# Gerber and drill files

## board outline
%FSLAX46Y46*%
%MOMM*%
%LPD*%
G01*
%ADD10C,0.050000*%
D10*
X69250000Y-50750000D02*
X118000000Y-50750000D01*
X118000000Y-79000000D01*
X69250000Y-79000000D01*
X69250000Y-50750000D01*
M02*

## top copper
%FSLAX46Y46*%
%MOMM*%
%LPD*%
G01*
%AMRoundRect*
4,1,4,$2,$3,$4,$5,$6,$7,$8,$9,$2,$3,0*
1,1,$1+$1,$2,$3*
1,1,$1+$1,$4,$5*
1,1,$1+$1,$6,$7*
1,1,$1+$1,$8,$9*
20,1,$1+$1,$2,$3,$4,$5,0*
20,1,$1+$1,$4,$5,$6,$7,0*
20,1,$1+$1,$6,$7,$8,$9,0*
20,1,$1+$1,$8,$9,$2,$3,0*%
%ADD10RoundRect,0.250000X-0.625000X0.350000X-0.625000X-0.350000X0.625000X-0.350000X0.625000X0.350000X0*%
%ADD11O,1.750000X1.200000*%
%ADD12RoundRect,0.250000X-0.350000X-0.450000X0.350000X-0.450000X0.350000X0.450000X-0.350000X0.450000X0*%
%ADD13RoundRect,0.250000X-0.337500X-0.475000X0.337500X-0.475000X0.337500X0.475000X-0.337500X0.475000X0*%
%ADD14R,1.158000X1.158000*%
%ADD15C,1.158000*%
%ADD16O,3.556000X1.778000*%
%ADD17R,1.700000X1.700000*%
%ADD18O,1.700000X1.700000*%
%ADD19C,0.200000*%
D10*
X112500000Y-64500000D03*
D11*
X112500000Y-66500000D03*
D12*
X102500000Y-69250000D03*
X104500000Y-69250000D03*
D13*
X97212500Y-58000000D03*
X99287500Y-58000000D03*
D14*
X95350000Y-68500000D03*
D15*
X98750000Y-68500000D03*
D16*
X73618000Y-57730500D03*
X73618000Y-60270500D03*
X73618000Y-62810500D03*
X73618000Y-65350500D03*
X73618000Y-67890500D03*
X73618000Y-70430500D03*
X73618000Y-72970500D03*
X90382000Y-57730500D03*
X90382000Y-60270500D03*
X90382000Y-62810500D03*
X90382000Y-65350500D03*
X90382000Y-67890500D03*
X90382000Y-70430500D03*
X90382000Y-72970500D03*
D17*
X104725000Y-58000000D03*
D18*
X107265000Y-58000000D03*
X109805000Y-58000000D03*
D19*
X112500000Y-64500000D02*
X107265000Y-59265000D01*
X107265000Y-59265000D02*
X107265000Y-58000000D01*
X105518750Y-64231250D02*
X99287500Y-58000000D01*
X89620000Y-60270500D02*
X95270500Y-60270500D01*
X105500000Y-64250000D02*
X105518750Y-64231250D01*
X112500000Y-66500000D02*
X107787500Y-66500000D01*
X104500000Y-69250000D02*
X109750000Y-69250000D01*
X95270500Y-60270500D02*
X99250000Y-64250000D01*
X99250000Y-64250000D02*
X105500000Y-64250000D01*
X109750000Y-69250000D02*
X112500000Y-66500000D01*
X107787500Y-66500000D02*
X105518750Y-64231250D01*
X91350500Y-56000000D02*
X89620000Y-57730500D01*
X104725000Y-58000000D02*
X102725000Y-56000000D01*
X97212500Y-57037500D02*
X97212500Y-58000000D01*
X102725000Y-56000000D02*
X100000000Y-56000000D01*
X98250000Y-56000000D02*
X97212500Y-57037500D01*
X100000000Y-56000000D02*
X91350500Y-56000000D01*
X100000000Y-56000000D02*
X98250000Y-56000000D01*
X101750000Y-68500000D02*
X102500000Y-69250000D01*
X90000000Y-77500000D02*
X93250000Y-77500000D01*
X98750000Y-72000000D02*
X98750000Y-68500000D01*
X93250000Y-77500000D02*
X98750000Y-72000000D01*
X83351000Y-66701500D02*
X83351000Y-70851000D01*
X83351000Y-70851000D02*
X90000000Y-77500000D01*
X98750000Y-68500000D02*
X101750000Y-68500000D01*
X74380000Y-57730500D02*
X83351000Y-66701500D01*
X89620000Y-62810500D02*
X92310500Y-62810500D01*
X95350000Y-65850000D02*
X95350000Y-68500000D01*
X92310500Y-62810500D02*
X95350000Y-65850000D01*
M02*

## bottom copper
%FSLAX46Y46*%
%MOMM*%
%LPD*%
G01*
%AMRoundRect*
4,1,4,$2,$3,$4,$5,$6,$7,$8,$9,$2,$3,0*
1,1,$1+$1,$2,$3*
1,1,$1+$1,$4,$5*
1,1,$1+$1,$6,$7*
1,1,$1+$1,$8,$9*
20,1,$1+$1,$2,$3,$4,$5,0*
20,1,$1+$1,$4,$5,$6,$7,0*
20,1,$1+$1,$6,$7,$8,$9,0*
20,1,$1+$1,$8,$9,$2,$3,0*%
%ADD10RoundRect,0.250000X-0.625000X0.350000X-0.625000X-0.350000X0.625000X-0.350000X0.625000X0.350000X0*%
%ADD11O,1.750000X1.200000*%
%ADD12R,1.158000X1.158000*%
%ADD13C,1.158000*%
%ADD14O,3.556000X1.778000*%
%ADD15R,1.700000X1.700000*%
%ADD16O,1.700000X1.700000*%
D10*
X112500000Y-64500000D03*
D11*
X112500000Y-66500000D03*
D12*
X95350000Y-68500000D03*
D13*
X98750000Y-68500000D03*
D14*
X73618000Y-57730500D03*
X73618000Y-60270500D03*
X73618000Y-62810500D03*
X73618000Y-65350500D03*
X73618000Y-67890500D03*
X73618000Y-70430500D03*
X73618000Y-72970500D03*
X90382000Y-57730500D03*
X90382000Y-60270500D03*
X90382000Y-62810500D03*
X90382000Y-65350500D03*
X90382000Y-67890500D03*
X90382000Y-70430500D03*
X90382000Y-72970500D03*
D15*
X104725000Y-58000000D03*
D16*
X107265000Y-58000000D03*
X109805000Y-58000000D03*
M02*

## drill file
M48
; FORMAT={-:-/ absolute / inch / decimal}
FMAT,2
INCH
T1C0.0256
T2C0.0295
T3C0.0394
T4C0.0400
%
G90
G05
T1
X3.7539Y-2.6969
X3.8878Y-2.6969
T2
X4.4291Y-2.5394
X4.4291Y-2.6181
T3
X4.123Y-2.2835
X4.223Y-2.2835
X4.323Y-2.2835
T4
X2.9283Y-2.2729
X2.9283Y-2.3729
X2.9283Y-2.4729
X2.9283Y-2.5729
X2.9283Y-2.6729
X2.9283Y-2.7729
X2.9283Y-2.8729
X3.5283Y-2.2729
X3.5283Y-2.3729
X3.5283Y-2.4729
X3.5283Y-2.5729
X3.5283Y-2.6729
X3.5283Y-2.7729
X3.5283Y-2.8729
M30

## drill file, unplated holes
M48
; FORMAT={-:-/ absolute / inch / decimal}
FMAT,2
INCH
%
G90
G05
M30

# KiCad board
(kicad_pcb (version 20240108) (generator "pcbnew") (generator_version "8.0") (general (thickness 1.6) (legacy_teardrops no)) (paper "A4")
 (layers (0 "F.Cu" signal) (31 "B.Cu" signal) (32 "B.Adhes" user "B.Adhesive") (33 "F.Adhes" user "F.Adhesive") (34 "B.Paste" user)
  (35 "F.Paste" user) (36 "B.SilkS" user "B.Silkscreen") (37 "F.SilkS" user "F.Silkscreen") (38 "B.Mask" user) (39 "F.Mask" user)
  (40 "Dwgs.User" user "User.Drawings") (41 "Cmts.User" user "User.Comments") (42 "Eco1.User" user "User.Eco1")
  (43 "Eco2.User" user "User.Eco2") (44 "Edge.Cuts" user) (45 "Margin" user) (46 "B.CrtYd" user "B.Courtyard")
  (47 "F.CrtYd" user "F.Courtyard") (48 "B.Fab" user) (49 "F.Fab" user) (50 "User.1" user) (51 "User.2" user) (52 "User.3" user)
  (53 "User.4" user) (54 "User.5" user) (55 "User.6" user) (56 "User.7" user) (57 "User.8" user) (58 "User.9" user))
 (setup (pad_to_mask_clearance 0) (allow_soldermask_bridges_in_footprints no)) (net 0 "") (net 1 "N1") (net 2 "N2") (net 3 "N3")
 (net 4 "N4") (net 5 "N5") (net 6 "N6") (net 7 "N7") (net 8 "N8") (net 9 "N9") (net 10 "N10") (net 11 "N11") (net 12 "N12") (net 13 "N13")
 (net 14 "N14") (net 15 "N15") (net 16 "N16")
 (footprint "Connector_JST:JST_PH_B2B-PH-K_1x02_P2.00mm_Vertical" (layer "F.Cu") (at 112.5 64.5 -90)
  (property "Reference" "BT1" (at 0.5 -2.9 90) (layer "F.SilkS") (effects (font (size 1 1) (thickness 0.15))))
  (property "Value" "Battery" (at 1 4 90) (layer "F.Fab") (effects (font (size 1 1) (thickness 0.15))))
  (pad "1" thru_hole roundrect (at 0 0 270) (size 1.2 1.75) (drill 0.75) (layers "*.Cu" "*.Mask") (remove_unused_layers no)
   (roundrect_rratio 0.208333) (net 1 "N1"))
  (pad "2" thru_hole oval (at 2 0 270) (size 1.2 1.75) (drill 0.75) (layers "*.Cu" "*.Mask") (remove_unused_layers no) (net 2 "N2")))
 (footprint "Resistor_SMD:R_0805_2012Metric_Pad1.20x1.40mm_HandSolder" (layer "F.Cu") (at 104 69.25)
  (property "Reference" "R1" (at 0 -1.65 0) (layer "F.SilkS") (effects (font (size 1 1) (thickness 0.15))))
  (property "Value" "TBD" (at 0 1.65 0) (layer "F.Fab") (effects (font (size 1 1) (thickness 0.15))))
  (pad "1" smd roundrect (at -1.5 0) (size 1.2 1.4) (layers "F.Cu" "F.Paste" "F.Mask") (roundrect_rratio 0.208333) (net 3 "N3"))
  (pad "2" smd roundrect (at 0.5 0) (size 1.2 1.4) (layers "F.Cu" "F.Paste" "F.Mask") (roundrect_rratio 0.208333) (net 2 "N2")))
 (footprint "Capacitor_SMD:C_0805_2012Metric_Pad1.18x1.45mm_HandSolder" (layer "F.Cu") (at 98.25 58)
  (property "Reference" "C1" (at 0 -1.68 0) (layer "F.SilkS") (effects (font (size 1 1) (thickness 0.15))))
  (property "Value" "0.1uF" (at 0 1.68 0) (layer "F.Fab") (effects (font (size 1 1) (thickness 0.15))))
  (pad "1" smd roundrect (at -1.0375 0) (size 1.175 1.45) (layers "F.Cu" "F.Paste" "F.Mask") (roundrect_rratio 0.212766) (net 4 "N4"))
  (pad "2" smd roundrect (at 1.0375 0) (size 1.175 1.45) (layers "F.Cu" "F.Paste" "F.Mask") (roundrect_rratio 0.212766) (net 2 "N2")))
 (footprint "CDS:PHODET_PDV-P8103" (layer "F.Cu") (at 97.05 68.5)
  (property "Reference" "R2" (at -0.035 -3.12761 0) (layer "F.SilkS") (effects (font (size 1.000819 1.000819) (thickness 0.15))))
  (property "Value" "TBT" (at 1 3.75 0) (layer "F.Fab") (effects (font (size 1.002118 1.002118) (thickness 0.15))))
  (pad "1" thru_hole rect (at -1.7 0) (size 1.158 1.158) (drill 0.65) (layers "*.Cu" "*.Mask") (remove_unused_layers no) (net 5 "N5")
   (solder_mask_margin 0.102))
  (pad "2" thru_hole circle (at 1.7 0) (size 1.158 1.158) (drill 0.65) (layers "*.Cu" "*.Mask") (remove_unused_layers no) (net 3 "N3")
   (solder_mask_margin 0.102)))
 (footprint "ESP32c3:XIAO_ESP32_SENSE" (layer "F.Cu") (at 82 65.3505)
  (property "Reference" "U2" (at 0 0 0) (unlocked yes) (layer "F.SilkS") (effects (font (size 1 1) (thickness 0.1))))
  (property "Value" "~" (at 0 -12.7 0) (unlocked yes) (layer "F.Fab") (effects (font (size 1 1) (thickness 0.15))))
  (pad "1" thru_hole oval (at -7.62 -7.62) (size 3.556 1.778) (drill 1.016 (offset -0.762 0)) (layers "*.Cu" "*.Mask")
   (remove_unused_layers no) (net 3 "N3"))
  (pad "2" thru_hole oval (at -7.62 -5.08) (size 3.556 1.778) (drill 1.016 (offset -0.762 0)) (layers "*.Cu" "*.Mask")
   (remove_unused_layers no) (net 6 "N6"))
  (pad "3" thru_hole oval (at -7.62 -2.54) (size 3.556 1.778) (drill 1.016 (offset -0.762 0)) (layers "*.Cu" "*.Mask")
   (remove_unused_layers no) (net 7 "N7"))
  (pad "4" thru_hole oval (at -7.62 0) (size 3.556 1.778) (drill 1.016 (offset -0.762 0)) (layers "*.Cu" "*.Mask") (remove_unused_layers no)
   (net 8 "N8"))
  (pad "5" thru_hole oval (at -7.62 2.54) (size 3.556 1.778) (drill 1.016 (offset -0.762 0)) (layers "*.Cu" "*.Mask")
   (remove_unused_layers no) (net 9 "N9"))
  (pad "6" thru_hole oval (at -7.62 5.08) (size 3.556 1.778) (drill 1.016 (offset -0.762 0)) (layers "*.Cu" "*.Mask")
   (remove_unused_layers no) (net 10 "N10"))
  (pad "7" thru_hole oval (at -7.62 7.62) (size 3.556 1.778) (drill 1.016 (offset -0.762 0)) (layers "*.Cu" "*.Mask")
   (remove_unused_layers no) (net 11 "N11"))
  (pad "8" thru_hole oval (at 7.62 -7.62) (size 3.556 1.778) (drill 1.016 (offset 0.762 0)) (layers "*.Cu" "*.Mask")
   (remove_unused_layers no) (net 4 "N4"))
  (pad "9" thru_hole oval (at 7.62 -5.08) (size 3.556 1.778) (drill 1.016 (offset 0.762 0)) (layers "*.Cu" "*.Mask")
   (remove_unused_layers no) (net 2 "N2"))
  (pad "10" thru_hole oval (at 7.62 -2.54) (size 3.556 1.778) (drill 1.016 (offset 0.762 0)) (layers "*.Cu" "*.Mask")
   (remove_unused_layers no) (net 5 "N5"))
  (pad "11" thru_hole oval (at 7.62 0) (size 3.556 1.778) (drill 1.016 (offset 0.762 0)) (layers "*.Cu" "*.Mask") (remove_unused_layers no)
   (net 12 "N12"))
  (pad "12" thru_hole oval (at 7.62 2.54) (size 3.556 1.778) (drill 1.016 (offset 0.762 0)) (layers "*.Cu" "*.Mask")
   (remove_unused_layers no) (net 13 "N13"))
  (pad "13" thru_hole oval (at 7.62 5.08) (size 3.556 1.778) (drill 1.016 (offset 0.762 0)) (layers "*.Cu" "*.Mask")
   (remove_unused_layers no) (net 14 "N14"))
  (pad "14" thru_hole oval (at 7.62 7.62) (size 3.556 1.778) (drill 1.016 (offset 0.762 0)) (layers "*.Cu" "*.Mask")
   (remove_unused_layers no) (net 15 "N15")))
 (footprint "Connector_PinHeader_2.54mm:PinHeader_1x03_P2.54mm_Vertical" (layer "F.Cu") (at 104.725 58 90)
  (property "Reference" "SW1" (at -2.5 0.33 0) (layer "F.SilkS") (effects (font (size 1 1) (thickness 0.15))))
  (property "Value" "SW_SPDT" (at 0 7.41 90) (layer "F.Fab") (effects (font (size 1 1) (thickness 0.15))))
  (pad "1" thru_hole rect (at 0 0 90) (size 1.7 1.7) (drill 1) (layers "*.Cu" "*.Mask") (remove_unused_layers no) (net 4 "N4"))
  (pad "2" thru_hole oval (at 0 2.54 90) (size 1.7 1.7) (drill 1) (layers "*.Cu" "*.Mask") (remove_unused_layers no) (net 1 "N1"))
  (pad "3" thru_hole oval (at 0 5.08 90) (size 1.7 1.7) (drill 1) (layers "*.Cu" "*.Mask") (remove_unused_layers no) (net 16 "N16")))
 (gr_rect (start 69.25 50.75) (end 118 79) (stroke (width 0.05) (type default)) (fill none) (layer "Edge.Cuts"))
 (segment (start 112.5 64.5) (end 107.265 59.265) (width 0.2) (layer "F.Cu") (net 1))
 (segment (start 107.265 59.265) (end 107.265 58) (width 0.2) (layer "F.Cu") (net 1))
 (segment (start 105.51875 64.23125) (end 99.2875 58) (width 0.2) (layer "F.Cu") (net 2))
 (segment (start 89.62 60.2705) (end 95.2705 60.2705) (width 0.2) (layer "F.Cu") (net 2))
 (segment (start 105.5 64.25) (end 105.51875 64.23125) (width 0.2) (layer "F.Cu") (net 2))
 (segment (start 112.5 66.5) (end 107.7875 66.5) (width 0.2) (layer "F.Cu") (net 2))
 (segment (start 104.5 69.25) (end 109.75 69.25) (width 0.2) (layer "F.Cu") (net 2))
 (segment (start 95.2705 60.2705) (end 99.25 64.25) (width 0.2) (layer "F.Cu") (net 2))
 (segment (start 99.25 64.25) (end 105.5 64.25) (width 0.2) (layer "F.Cu") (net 2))
 (segment (start 109.75 69.25) (end 112.5 66.5) (width 0.2) (layer "F.Cu") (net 2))
 (segment (start 107.7875 66.5) (end 105.51875 64.23125) (width 0.2) (layer "F.Cu") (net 2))
 (segment (start 91.3505 56) (end 89.62 57.7305) (width 0.2) (layer "F.Cu") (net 4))
 (segment (start 104.725 58) (end 102.725 56) (width 0.2) (layer "F.Cu") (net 4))
 (segment (start 97.2125 57.0375) (end 97.2125 58) (width 0.2) (layer "F.Cu") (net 4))
 (segment (start 102.725 56) (end 100 56) (width 0.2) (layer "F.Cu") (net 4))
 (segment (start 98.25 56) (end 97.2125 57.0375) (width 0.2) (layer "F.Cu") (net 4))
 (segment (start 100 56) (end 91.3505 56) (width 0.2) (layer "F.Cu") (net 4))
 (segment (start 100 56) (end 98.25 56) (width 0.2) (layer "F.Cu") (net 4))
 (segment (start 101.75 68.5) (end 102.5 69.25) (width 0.2) (layer "F.Cu") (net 3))
 (segment (start 90 77.5) (end 93.25 77.5) (width 0.2) (layer "F.Cu") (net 3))
 (segment (start 98.75 72) (end 98.75 68.5) (width 0.2) (layer "F.Cu") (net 3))
 (segment (start 93.25 77.5) (end 98.75 72) (width 0.2) (layer "F.Cu") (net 3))
 (segment (start 83.351 66.7015) (end 83.351 70.851) (width 0.2) (layer "F.Cu") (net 3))
 (segment (start 83.351 70.851) (end 90 77.5) (width 0.2) (layer "F.Cu") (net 3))
 (segment (start 98.75 68.5) (end 101.75 68.5) (width 0.2) (layer "F.Cu") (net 3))
 (segment (start 74.38 57.7305) (end 83.351 66.7015) (width 0.2) (layer "F.Cu") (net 3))
 (segment (start 89.62 62.8105) (end 92.3105 62.8105) (width 0.2) (layer "F.Cu") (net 5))
 (segment (start 95.35 65.85) (end 95.35 68.5) (width 0.2) (layer "F.Cu") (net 5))
 (segment (start 92.3105 62.8105) (end 95.35 65.85) (width 0.2) (layer "F.Cu") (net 5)))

